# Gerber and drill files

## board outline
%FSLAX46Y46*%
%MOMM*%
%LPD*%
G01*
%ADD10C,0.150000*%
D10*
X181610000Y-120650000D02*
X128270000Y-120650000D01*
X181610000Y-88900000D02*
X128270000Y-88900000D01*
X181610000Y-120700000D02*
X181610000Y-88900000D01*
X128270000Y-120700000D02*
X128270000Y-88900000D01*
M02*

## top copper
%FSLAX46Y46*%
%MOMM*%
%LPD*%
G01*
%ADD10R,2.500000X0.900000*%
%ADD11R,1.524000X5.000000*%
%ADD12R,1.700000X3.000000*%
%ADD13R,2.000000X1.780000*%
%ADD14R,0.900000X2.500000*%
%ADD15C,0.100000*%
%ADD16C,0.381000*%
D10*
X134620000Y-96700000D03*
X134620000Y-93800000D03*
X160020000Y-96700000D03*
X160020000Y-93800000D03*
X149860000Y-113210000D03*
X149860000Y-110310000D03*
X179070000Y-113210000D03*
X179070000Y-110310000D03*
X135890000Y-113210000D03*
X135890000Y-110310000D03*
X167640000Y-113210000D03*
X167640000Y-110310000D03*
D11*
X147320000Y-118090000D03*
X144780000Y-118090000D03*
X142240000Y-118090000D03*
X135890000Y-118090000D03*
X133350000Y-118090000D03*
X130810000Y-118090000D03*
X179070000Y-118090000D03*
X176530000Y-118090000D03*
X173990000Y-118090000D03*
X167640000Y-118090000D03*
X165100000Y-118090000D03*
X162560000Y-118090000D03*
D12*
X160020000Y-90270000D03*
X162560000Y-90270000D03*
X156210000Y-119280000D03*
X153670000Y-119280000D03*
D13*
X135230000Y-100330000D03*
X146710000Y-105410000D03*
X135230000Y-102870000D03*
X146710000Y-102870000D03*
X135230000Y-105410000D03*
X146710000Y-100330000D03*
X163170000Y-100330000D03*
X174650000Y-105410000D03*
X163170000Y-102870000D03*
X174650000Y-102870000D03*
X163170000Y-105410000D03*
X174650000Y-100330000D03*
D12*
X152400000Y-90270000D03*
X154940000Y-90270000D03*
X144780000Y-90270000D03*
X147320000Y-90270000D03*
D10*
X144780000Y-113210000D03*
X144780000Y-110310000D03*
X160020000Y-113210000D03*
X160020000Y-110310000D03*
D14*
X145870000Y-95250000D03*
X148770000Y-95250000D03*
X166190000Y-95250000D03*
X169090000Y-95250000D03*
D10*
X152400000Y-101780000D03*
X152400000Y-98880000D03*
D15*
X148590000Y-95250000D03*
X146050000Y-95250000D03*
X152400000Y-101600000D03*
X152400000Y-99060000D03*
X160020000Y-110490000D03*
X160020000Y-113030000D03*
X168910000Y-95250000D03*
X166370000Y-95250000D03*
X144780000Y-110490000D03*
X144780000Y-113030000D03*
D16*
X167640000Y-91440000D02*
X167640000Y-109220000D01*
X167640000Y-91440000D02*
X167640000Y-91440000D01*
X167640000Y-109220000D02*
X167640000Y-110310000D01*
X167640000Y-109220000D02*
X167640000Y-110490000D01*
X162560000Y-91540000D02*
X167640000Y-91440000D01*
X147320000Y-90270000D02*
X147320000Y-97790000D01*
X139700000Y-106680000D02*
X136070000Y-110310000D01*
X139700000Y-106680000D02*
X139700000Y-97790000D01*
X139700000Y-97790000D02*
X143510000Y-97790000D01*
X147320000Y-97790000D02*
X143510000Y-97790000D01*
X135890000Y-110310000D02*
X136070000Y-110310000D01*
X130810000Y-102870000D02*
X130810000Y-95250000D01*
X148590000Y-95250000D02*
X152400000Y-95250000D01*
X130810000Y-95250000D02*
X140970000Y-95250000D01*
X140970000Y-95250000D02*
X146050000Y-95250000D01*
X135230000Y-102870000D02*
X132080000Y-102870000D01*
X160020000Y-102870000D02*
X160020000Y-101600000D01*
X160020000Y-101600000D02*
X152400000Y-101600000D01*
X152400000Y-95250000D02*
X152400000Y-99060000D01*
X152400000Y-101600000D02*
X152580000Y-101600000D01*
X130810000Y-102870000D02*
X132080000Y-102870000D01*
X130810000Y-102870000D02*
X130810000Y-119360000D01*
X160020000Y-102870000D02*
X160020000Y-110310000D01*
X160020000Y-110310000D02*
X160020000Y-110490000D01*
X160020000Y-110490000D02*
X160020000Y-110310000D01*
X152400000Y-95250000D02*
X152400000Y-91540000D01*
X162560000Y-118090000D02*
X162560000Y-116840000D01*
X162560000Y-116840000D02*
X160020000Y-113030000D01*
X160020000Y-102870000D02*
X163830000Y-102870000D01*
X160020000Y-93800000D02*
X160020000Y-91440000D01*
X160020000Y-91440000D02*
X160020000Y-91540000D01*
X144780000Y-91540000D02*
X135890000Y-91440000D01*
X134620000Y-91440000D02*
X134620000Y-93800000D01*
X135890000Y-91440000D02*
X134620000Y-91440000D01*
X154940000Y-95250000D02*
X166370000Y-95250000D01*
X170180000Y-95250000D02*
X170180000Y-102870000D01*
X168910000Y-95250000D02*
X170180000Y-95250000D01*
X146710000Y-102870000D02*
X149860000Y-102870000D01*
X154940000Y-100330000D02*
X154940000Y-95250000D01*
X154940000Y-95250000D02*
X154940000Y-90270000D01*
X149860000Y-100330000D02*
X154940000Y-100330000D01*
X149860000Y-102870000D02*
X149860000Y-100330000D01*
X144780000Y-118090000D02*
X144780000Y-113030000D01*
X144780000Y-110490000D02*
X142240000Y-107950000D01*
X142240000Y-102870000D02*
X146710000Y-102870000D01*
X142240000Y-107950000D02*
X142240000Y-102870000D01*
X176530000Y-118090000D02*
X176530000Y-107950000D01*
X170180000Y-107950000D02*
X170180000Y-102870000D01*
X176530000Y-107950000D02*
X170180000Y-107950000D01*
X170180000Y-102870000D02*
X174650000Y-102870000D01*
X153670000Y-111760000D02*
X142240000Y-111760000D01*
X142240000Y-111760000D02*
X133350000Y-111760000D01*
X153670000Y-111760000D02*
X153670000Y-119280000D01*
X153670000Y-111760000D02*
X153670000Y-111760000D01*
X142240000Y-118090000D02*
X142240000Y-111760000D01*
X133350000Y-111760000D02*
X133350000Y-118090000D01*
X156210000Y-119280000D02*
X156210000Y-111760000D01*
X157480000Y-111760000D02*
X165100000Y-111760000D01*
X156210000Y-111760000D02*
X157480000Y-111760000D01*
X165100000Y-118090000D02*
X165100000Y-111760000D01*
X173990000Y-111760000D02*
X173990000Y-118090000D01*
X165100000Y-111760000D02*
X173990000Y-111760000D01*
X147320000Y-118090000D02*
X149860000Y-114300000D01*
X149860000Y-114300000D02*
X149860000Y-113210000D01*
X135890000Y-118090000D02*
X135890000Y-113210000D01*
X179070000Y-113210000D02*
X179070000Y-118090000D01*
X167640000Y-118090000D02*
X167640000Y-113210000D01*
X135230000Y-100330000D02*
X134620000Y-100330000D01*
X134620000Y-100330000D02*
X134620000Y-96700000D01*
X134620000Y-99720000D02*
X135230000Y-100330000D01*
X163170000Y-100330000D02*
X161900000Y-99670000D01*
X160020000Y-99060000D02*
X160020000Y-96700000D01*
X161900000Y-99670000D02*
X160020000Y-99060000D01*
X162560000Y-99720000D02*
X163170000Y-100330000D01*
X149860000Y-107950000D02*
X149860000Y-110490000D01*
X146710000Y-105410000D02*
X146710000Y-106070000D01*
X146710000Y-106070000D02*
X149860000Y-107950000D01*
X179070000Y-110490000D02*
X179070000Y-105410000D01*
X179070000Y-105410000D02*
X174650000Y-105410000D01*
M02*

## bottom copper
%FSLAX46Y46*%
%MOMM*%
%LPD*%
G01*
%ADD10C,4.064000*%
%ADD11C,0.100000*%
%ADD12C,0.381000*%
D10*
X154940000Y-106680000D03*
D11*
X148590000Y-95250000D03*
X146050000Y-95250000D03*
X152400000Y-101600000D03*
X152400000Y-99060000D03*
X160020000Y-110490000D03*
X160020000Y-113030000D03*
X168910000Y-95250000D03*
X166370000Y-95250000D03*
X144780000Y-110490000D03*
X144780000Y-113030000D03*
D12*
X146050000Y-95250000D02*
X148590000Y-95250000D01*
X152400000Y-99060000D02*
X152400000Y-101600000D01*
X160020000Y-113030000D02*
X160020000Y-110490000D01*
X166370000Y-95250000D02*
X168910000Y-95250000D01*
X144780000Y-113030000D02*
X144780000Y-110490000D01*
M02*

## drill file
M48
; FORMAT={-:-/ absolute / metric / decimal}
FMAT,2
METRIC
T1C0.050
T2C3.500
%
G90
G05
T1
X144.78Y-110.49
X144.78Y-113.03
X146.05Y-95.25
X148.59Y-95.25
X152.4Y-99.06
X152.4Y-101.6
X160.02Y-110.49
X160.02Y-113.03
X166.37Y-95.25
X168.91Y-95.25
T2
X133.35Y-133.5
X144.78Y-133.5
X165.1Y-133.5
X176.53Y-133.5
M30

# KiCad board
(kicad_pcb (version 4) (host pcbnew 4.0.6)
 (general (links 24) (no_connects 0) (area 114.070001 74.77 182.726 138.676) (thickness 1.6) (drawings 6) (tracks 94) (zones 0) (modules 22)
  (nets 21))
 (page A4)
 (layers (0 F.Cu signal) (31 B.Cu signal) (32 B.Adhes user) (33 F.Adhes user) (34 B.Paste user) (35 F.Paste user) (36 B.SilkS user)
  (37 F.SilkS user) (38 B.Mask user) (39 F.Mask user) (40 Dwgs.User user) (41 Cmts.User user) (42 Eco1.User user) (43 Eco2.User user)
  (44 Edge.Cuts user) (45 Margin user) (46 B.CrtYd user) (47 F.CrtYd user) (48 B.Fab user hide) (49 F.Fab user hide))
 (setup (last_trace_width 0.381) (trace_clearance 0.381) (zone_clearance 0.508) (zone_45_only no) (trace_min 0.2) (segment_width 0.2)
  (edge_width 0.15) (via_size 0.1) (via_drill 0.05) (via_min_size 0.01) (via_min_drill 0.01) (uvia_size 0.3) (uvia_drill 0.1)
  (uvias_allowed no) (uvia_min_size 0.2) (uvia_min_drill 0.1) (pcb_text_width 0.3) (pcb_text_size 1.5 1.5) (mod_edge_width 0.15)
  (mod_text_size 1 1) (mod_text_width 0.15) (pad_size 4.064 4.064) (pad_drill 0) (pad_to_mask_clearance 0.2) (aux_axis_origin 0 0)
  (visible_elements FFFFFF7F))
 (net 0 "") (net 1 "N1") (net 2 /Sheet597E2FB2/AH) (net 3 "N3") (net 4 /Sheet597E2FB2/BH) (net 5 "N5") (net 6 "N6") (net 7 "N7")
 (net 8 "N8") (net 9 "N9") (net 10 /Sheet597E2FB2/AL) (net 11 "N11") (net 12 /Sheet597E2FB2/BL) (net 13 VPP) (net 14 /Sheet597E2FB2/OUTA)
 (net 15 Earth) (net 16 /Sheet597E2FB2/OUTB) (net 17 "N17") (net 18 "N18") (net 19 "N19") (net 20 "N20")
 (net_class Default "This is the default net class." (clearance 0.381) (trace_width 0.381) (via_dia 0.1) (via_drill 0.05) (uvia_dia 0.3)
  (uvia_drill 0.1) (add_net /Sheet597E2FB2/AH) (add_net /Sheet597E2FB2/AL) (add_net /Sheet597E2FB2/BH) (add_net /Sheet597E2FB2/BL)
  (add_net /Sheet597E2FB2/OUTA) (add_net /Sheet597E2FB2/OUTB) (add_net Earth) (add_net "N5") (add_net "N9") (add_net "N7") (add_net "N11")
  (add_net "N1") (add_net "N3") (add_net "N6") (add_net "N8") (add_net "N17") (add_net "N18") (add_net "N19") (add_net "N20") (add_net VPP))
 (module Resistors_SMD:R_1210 (layer F.Cu) (at 134.62 95.25 90)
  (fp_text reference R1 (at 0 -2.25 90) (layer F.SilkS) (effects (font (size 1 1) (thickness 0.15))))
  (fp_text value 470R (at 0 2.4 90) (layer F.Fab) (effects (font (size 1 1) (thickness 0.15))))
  (pad 1 smd rect (at -1.45 0 90) (size 0.9 2.5) (layers F.Cu F.Paste F.Mask) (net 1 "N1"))
  (pad 2 smd rect (at 1.45 0 90) (size 0.9 2.5) (layers F.Cu F.Paste F.Mask) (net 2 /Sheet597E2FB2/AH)))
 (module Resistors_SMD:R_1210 (layer F.Cu) (at 160.02 95.25 90)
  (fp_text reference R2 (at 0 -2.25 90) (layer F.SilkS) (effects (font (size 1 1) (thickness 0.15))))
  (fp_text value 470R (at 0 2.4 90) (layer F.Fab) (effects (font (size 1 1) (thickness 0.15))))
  (pad 1 smd rect (at -1.45 0 90) (size 0.9 2.5) (layers F.Cu F.Paste F.Mask) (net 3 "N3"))
  (pad 2 smd rect (at 1.45 0 90) (size 0.9 2.5) (layers F.Cu F.Paste F.Mask) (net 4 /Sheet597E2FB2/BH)))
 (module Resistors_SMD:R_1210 (layer F.Cu) (at 149.86 111.76 90)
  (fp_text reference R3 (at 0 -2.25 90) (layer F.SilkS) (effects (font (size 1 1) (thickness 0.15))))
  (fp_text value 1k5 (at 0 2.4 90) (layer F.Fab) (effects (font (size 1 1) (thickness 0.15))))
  (pad 1 smd rect (at -1.45 0 90) (size 0.9 2.5) (layers F.Cu F.Paste F.Mask) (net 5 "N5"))
  (pad 2 smd rect (at 1.45 0 90) (size 0.9 2.5) (layers F.Cu F.Paste F.Mask) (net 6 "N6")))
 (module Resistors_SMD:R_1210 (layer F.Cu) (at 179.07 111.76 90)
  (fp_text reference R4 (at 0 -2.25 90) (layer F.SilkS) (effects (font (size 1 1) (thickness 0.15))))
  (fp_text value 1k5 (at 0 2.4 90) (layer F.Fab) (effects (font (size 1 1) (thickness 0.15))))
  (pad 1 smd rect (at -1.45 0 90) (size 0.9 2.5) (layers F.Cu F.Paste F.Mask) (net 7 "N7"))
  (pad 2 smd rect (at 1.45 0 90) (size 0.9 2.5) (layers F.Cu F.Paste F.Mask) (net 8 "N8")))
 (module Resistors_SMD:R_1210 (layer F.Cu) (at 135.89 111.76 90)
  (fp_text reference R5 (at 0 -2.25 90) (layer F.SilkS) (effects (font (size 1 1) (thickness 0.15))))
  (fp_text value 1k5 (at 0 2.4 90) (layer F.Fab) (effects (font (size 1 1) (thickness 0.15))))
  (pad 1 smd rect (at -1.45 0 90) (size 0.9 2.5) (layers F.Cu F.Paste F.Mask) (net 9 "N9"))
  (pad 2 smd rect (at 1.45 0 90) (size 0.9 2.5) (layers F.Cu F.Paste F.Mask) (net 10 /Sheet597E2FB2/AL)))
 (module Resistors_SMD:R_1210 (layer F.Cu) (at 167.64 111.76 90)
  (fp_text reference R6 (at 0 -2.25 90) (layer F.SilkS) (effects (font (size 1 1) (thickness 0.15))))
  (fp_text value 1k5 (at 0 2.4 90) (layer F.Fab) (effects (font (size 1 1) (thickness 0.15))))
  (pad 1 smd rect (at -1.45 0 90) (size 0.9 2.5) (layers F.Cu F.Paste F.Mask) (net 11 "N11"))
  (pad 2 smd rect (at 1.45 0 90) (size 0.9 2.5) (layers F.Cu F.Paste F.Mask) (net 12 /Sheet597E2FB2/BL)))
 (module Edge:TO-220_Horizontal (layer F.Cu) (at 147.32 116.84 180)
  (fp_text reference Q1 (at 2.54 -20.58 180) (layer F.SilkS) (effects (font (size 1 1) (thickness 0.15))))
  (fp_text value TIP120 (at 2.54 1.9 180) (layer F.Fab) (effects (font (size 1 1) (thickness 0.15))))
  (pad 1 smd rect (at 0 -1.25 180) (size 1.524 5) (layers F.Cu F.Paste F.Mask) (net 5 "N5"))
  (pad 2 smd rect (at 2.54 -1.25 180) (size 1.524 5) (layers F.Cu F.Paste F.Mask) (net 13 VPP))
  (pad None np_thru_hole oval (at 2.54 -16.66 180) (size 3.5 3.5) (drill 3.5) (layers *.Cu *.Mask))
  (pad 3 smd rect (at 5.08 -1.25 180) (size 1.524 5) (layers F.Cu F.Paste F.Mask) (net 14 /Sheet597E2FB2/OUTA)))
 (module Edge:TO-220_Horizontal (layer F.Cu) (at 135.89 116.84 180)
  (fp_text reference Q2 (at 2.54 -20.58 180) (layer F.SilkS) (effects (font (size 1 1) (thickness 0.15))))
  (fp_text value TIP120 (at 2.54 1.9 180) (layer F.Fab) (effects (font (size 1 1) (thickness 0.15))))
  (pad 1 smd rect (at 0 -1.25 180) (size 1.524 5) (layers F.Cu F.Paste F.Mask) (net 9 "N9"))
  (pad 2 smd rect (at 2.54 -1.25 180) (size 1.524 5) (layers F.Cu F.Paste F.Mask) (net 14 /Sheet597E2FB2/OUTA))
  (pad None np_thru_hole oval (at 2.54 -16.66 180) (size 3.5 3.5) (drill 3.5) (layers *.Cu *.Mask))
  (pad 3 smd rect (at 5.08 -1.25 180) (size 1.524 5) (layers F.Cu F.Paste F.Mask) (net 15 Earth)))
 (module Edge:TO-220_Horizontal (layer F.Cu) (at 179.07 116.84 180)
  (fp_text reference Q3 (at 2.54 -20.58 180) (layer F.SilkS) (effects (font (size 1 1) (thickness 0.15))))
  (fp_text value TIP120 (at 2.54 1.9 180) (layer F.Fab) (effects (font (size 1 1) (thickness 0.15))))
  (pad 1 smd rect (at 0 -1.25 180) (size 1.524 5) (layers F.Cu F.Paste F.Mask) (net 7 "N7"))
  (pad 2 smd rect (at 2.54 -1.25 180) (size 1.524 5) (layers F.Cu F.Paste F.Mask) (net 13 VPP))
  (pad None np_thru_hole oval (at 2.54 -16.66 180) (size 3.5 3.5) (drill 3.5) (layers *.Cu *.Mask))
  (pad 3 smd rect (at 5.08 -1.25 180) (size 1.524 5) (layers F.Cu F.Paste F.Mask) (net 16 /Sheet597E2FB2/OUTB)))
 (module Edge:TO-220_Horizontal (layer F.Cu) (at 167.64 116.84 180)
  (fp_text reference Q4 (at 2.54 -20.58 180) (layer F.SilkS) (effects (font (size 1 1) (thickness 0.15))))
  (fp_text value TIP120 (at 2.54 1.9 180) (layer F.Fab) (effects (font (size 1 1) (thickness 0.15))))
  (pad 1 smd rect (at 0 -1.25 180) (size 1.524 5) (layers F.Cu F.Paste F.Mask) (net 11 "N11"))
  (pad 2 smd rect (at 2.54 -1.25 180) (size 1.524 5) (layers F.Cu F.Paste F.Mask) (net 16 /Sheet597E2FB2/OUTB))
  (pad None np_thru_hole oval (at 2.54 -16.66 180) (size 3.5 3.5) (drill 3.5) (layers *.Cu *.Mask))
  (pad 3 smd rect (at 5.08 -1.25 180) (size 1.524 5) (layers F.Cu F.Paste F.Mask) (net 15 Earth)))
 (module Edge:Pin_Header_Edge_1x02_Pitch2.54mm (layer F.Cu) (at 160.02 90.17 90)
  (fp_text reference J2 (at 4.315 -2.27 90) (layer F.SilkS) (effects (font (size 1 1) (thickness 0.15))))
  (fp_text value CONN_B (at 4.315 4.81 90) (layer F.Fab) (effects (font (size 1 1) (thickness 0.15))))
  (pad 1 smd rect (at -0.1 0 90) (size 3 1.7) (layers F.Cu F.Paste F.Mask) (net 4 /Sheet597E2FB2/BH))
  (pad 2 smd rect (at -0.1 2.54 90) (size 3 1.7) (layers F.Cu F.Paste F.Mask) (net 12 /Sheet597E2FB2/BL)))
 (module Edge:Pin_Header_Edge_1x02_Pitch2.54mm (layer F.Cu) (at 156.21 119.38 270)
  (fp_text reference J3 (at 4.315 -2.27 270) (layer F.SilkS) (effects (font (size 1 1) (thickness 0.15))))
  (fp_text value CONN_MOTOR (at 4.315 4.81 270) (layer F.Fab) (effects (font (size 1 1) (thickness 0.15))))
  (pad 1 smd rect (at -0.1 0 270) (size 3 1.7) (layers F.Cu F.Paste F.Mask) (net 16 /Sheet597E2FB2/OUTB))
  (pad 2 smd rect (at -0.1 2.54 270) (size 3 1.7) (layers F.Cu F.Paste F.Mask) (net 14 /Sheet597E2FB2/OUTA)))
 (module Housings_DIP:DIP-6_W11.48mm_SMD (layer F.Cu) (at 140.97 102.87)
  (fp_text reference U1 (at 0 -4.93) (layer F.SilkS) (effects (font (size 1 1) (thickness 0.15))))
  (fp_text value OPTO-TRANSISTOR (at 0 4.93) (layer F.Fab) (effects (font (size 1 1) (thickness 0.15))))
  (pad 1 smd rect (at -5.74 -2.54) (size 2 1.78) (layers F.Cu F.Mask) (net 1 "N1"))
  (pad 4 smd rect (at 5.74 2.54) (size 2 1.78) (layers F.Cu F.Mask) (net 6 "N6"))
  (pad 2 smd rect (at -5.74 0) (size 2 1.78) (layers F.Cu F.Mask) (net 15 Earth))
  (pad 5 smd rect (at 5.74 0) (size 2 1.78) (layers F.Cu F.Mask) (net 13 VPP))
  (pad 3 smd rect (at -5.74 2.54) (size 2 1.78) (layers F.Cu F.Mask) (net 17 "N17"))
  (pad 6 smd rect (at 5.74 -2.54) (size 2 1.78) (layers F.Cu F.Mask) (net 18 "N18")))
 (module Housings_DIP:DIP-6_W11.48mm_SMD (layer F.Cu) (at 168.91 102.87)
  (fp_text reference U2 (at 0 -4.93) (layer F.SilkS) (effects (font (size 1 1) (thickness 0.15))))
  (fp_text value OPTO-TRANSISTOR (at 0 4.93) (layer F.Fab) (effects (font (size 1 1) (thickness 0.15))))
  (pad 1 smd rect (at -5.74 -2.54) (size 2 1.78) (layers F.Cu F.Mask) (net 3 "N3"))
  (pad 4 smd rect (at 5.74 2.54) (size 2 1.78) (layers F.Cu F.Mask) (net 8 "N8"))
  (pad 2 smd rect (at -5.74 0) (size 2 1.78) (layers F.Cu F.Mask) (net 15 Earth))
  (pad 5 smd rect (at 5.74 0) (size 2 1.78) (layers F.Cu F.Mask) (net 13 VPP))
  (pad 3 smd rect (at -5.74 2.54) (size 2 1.78) (layers F.Cu F.Mask) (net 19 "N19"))
  (pad 6 smd rect (at 5.74 -2.54) (size 2 1.78) (layers F.Cu F.Mask) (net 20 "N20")))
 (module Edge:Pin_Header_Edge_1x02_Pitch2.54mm (layer F.Cu) (at 152.4 90.17 90)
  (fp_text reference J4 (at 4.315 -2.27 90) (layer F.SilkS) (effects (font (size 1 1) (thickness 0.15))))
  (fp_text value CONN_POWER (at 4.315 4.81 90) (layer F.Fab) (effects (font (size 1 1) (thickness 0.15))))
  (pad 1 smd rect (at -0.1 0 90) (size 3 1.7) (layers F.Cu F.Paste F.Mask) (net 15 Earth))
  (pad 2 smd rect (at -0.1 2.54 90) (size 3 1.7) (layers F.Cu F.Paste F.Mask) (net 13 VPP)))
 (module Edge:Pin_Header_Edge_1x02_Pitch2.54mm (layer F.Cu) (at 144.78 90.17 90)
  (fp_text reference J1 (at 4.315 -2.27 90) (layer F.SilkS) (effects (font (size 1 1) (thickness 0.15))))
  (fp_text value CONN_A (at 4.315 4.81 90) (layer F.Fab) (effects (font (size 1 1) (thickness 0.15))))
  (pad 1 smd rect (at -0.1 0 90) (size 3 1.7) (layers F.Cu F.Paste F.Mask) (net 2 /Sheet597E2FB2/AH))
  (pad 2 smd rect (at -0.1 2.54 90) (size 3 1.7) (layers F.Cu F.Paste F.Mask) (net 10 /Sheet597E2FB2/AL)))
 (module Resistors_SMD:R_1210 (layer F.Cu) (at 144.78 111.76 90)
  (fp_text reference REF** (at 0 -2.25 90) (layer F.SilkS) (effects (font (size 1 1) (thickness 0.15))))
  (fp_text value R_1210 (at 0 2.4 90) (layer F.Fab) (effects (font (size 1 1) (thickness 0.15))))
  (pad 1 smd rect (at -1.45 0 90) (size 0.9 2.5) (layers F.Cu F.Paste F.Mask))
  (pad 2 smd rect (at 1.45 0 90) (size 0.9 2.5) (layers F.Cu F.Paste F.Mask)))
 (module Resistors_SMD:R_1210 (layer F.Cu) (at 160.02 111.76 90)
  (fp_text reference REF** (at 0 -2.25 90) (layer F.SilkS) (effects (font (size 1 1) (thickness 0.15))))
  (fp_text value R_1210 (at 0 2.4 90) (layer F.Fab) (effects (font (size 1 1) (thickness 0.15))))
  (pad 1 smd rect (at -1.45 0 90) (size 0.9 2.5) (layers F.Cu F.Paste F.Mask))
  (pad 2 smd rect (at 1.45 0 90) (size 0.9 2.5) (layers F.Cu F.Paste F.Mask)))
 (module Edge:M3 (layer F.Cu) (at 154.94 106.68)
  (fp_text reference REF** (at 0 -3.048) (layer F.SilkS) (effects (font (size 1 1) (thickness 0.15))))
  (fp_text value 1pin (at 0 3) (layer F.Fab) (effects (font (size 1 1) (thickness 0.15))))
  (pad 1 smd circle (at 0 0) (size 4.064 4.064) (layers B.Cu F.Paste F.Mask)))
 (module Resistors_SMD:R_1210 (layer F.Cu) (at 147.32 95.25)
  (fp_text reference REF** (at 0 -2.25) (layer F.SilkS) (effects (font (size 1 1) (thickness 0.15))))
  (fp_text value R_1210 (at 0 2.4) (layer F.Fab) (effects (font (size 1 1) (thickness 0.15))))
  (pad 1 smd rect (at -1.45 0) (size 0.9 2.5) (layers F.Cu F.Paste F.Mask))
  (pad 2 smd rect (at 1.45 0) (size 0.9 2.5) (layers F.Cu F.Paste F.Mask)))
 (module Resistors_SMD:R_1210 (layer F.Cu) (at 167.64 95.25)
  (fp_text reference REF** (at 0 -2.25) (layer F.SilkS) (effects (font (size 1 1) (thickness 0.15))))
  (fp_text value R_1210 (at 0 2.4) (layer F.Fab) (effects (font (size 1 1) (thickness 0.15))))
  (pad 1 smd rect (at -1.45 0) (size 0.9 2.5) (layers F.Cu F.Paste F.Mask))
  (pad 2 smd rect (at 1.45 0) (size 0.9 2.5) (layers F.Cu F.Paste F.Mask)))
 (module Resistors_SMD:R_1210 (layer F.Cu) (at 152.4 100.33 90)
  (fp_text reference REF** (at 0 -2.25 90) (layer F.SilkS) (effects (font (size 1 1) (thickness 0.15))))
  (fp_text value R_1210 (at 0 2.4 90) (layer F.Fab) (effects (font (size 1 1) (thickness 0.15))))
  (pad 1 smd rect (at -1.45 0 90) (size 0.9 2.5) (layers F.Cu F.Paste F.Mask))
  (pad 2 smd rect (at 1.45 0 90) (size 0.9 2.5) (layers F.Cu F.Paste F.Mask)))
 (gr_line (start 181.61 120.65) (end 128.27 120.65) (angle 90) (layer Edge.Cuts) (width 0.15))
 (gr_line (start 181.61 88.9) (end 128.27 88.9) (angle 90) (layer Edge.Cuts) (width 0.15))
 (gr_line (start 181.61 120.7) (end 181.61 88.9) (angle 90) (layer Edge.Cuts) (width 0.15))
 (gr_line (start 128.27 120.7) (end 128.27 88.9) (angle 90) (layer Edge.Cuts) (width 0.15))
 (segment (start 167.64 91.44) (end 167.64 109.22) (width 0.381) (layer F.Cu) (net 12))
 (segment (start 167.64 91.44) (end 167.64 91.44) (width 0.381) (layer F.Cu) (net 12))
 (segment (start 167.64 109.22) (end 167.64 110.31) (width 0.381) (layer F.Cu) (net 12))
 (segment (start 167.64 109.22) (end 167.64 110.49) (width 0.381) (layer F.Cu) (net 12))
 (segment (start 162.56 91.54) (end 167.64 91.44) (width 0.381) (layer F.Cu) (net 12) (status 10))
 (segment (start 147.32 90.27) (end 147.32 97.79) (width 0.381) (layer F.Cu) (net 10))
 (segment (start 139.7 106.68) (end 136.07 110.31) (width 0.381) (layer F.Cu) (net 10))
 (segment (start 139.7 106.68) (end 139.7 97.79) (width 0.381) (layer F.Cu) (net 10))
 (segment (start 139.7 97.79) (end 143.51 97.79) (width 0.381) (layer F.Cu) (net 10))
 (segment (start 147.32 97.79) (end 143.51 97.79) (width 0.381) (layer F.Cu) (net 10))
 (segment (start 135.89 110.31) (end 136.07 110.31) (width 0.381) (layer F.Cu) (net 10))
 (segment (start 130.81 102.87) (end 130.81 95.25) (width 0.381) (layer F.Cu) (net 15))
 (via (at 148.59 95.25) (size 0.1) (drill 0.05) (layers F.Cu B.Cu) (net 15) (status 30))
 (segment (start 148.59 95.25) (end 152.4 95.25) (width 0.381) (layer F.Cu) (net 15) (status 10))
 (segment (start 130.81 95.25) (end 140.97 95.25) (width 0.381) (layer F.Cu) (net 15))
 (segment (start 140.97 95.25) (end 146.05 95.25) (width 0.381) (layer F.Cu) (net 15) (status 20))
 (via (at 146.05 95.25) (size 0.1) (drill 0.05) (layers F.Cu B.Cu) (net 15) (status 30))
 (segment (start 146.05 95.25) (end 148.59 95.25) (width 0.381) (layer B.Cu) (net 15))
 (segment (start 135.23 102.87) (end 132.08 102.87) (width 0.381) (layer F.Cu) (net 15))
 (segment (start 160.02 102.87) (end 160.02 101.6) (width 0.381) (layer F.Cu) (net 15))
 (segment (start 160.02 101.6) (end 152.4 101.6) (width 0.381) (layer F.Cu) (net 15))
 (segment (start 152.4 95.25) (end 152.4 99.06) (width 0.381) (layer F.Cu) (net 15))
 (via (at 152.4 101.6) (size 0.1) (drill 0.05) (layers F.Cu B.Cu) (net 15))
 (segment (start 152.4 99.06) (end 152.4 101.6) (width 0.381) (layer B.Cu) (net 15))
 (via (at 152.4 99.06) (size 0.1) (drill 0.05) (layers F.Cu B.Cu) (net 15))
 (segment (start 152.4 101.6) (end 152.58 101.6) (width 0.381) (layer F.Cu) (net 15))
 (segment (start 130.81 102.87) (end 132.08 102.87) (width 0.381) (layer F.Cu) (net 15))
 (segment (start 130.81 102.87) (end 130.81 119.36) (width 0.381) (layer F.Cu) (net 15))
 (segment (start 160.02 102.87) (end 160.02 110.31) (width 0.381) (layer F.Cu) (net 15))
 (segment (start 160.02 110.31) (end 160.02 110.49) (width 0.381) (layer F.Cu) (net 15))
 (segment (start 160.02 110.49) (end 160.02 110.31) (width 0.381) (layer F.Cu) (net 15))
 (segment (start 152.4 95.25) (end 152.4 91.54) (width 0.381) (layer F.Cu) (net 15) (status 20))
 (segment (start 162.56 118.09) (end 162.56 116.84) (width 0.381) (layer F.Cu) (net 15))
 (segment (start 162.56 116.84) (end 160.02 113.03) (width 0.381) (layer F.Cu) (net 15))
 (via (at 160.02 110.49) (size 0.1) (drill 0.05) (layers F.Cu B.Cu) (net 15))
 (segment (start 160.02 113.03) (end 160.02 110.49) (width 0.381) (layer B.Cu) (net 15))
 (via (at 160.02 113.03) (size 0.1) (drill 0.05) (layers F.Cu B.Cu) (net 15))
 (segment (start 160.02 102.87) (end 163.83 102.87) (width 0.381) (layer F.Cu) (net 15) (status 20))
 (segment (start 160.02 93.8) (end 160.02 91.44) (width 0.381) (layer F.Cu) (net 4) (status 10))
 (segment (start 160.02 91.44) (end 160.02 91.54) (width 0.381) (layer F.Cu) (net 4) (status 30))
 (segment (start 144.78 91.54) (end 135.89 91.44) (width 0.381) (layer F.Cu) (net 2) (status 10))
 (segment (start 134.62 91.44) (end 134.62 93.8) (width 0.381) (layer F.Cu) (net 2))
 (segment (start 135.89 91.44) (end 134.62 91.44) (width 0.381) (layer F.Cu) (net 2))
 (segment (start 154.94 95.25) (end 166.37 95.25) (width 0.381) (layer F.Cu) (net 13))
 (segment (start 170.18 95.25) (end 170.18 102.87) (width 0.381) (layer F.Cu) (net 13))
 (segment (start 168.91 95.25) (end 170.18 95.25) (width 0.381) (layer F.Cu) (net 13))
 (via (at 168.91 95.25) (size 0.1) (drill 0.05) (layers F.Cu B.Cu) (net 13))
 (segment (start 166.37 95.25) (end 168.91 95.25) (width 0.381) (layer B.Cu) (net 13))
 (via (at 166.37 95.25) (size 0.1) (drill 0.05) (layers F.Cu B.Cu) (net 13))
 (segment (start 146.71 102.87) (end 149.86 102.87) (width 0.381) (layer F.Cu) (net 13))
 (segment (start 154.94 100.33) (end 154.94 95.25) (width 0.381) (layer F.Cu) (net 13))
 (segment (start 154.94 95.25) (end 154.94 90.27) (width 0.381) (layer F.Cu) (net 13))
 (segment (start 149.86 100.33) (end 154.94 100.33) (width 0.381) (layer F.Cu) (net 13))
 (segment (start 149.86 102.87) (end 149.86 100.33) (width 0.381) (layer F.Cu) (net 13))
 (segment (start 144.78 118.09) (end 144.78 113.03) (width 0.381) (layer F.Cu) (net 13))
 (via (at 144.78 110.49) (size 0.1) (drill 0.05) (layers F.Cu B.Cu) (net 13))
 (segment (start 144.78 113.03) (end 144.78 110.49) (width 0.381) (layer B.Cu) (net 13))
 (via (at 144.78 113.03) (size 0.1) (drill 0.05) (layers F.Cu B.Cu) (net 13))
 (segment (start 144.78 110.49) (end 142.24 107.95) (width 0.381) (layer F.Cu) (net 13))
 (segment (start 142.24 102.87) (end 146.71 102.87) (width 0.381) (layer F.Cu) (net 13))
 (segment (start 142.24 107.95) (end 142.24 102.87) (width 0.381) (layer F.Cu) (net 13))
 (segment (start 176.53 118.09) (end 176.53 107.95) (width 0.381) (layer F.Cu) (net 13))
 (segment (start 170.18 107.95) (end 170.18 102.87) (width 0.381) (layer F.Cu) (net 13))
 (segment (start 176.53 107.95) (end 170.18 107.95) (width 0.381) (layer F.Cu) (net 13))
 (segment (start 170.18 102.87) (end 174.65 102.87) (width 0.381) (layer F.Cu) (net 13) (status 20))
 (segment (start 153.67 111.76) (end 142.24 111.76) (width 0.381) (layer F.Cu) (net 14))
 (segment (start 142.24 111.76) (end 133.35 111.76) (width 0.381) (layer F.Cu) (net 14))
 (segment (start 153.67 111.76) (end 153.67 119.28) (width 0.381) (layer F.Cu) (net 14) (status 20))
 (segment (start 153.67 111.76) (end 153.67 111.76) (width 0.381) (layer F.Cu) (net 14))
 (segment (start 142.24 118.09) (end 142.24 111.76) (width 0.381) (layer F.Cu) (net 14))
 (segment (start 133.35 111.76) (end 133.35 118.09) (width 0.381) (layer F.Cu) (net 14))
 (segment (start 156.21 119.28) (end 156.21 111.76) (width 0.381) (layer F.Cu) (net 16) (status 10))
 (segment (start 157.48 111.76) (end 165.1 111.76) (width 0.381) (layer F.Cu) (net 16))
 (segment (start 156.21 111.76) (end 157.48 111.76) (width 0.381) (layer F.Cu) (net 16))
 (segment (start 165.1 118.09) (end 165.1 111.76) (width 0.381) (layer F.Cu) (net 16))
 (segment (start 173.99 111.76) (end 173.99 118.09) (width 0.381) (layer F.Cu) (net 16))
 (segment (start 165.1 111.76) (end 173.99 111.76) (width 0.381) (layer F.Cu) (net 16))
 (segment (start 147.32 118.09) (end 149.86 114.3) (width 0.381) (layer F.Cu) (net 5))
 (segment (start 149.86 114.3) (end 149.86 113.21) (width 0.381) (layer F.Cu) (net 5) (status 20))
 (segment (start 135.89 118.09) (end 135.89 113.21) (width 0.381) (layer F.Cu) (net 9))
 (segment (start 179.07 113.21) (end 179.07 118.09) (width 0.381) (layer F.Cu) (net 7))
 (segment (start 167.64 118.09) (end 167.64 113.21) (width 0.381) (layer F.Cu) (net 11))
 (segment (start 135.23 100.33) (end 134.62 100.33) (width 0.381) (layer F.Cu) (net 1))
 (segment (start 134.62 100.33) (end 134.62 96.7) (width 0.381) (layer F.Cu) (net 1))
 (segment (start 134.62 99.72) (end 135.23 100.33) (width 0.381) (layer F.Cu) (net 1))
 (segment (start 163.17 100.33) (end 161.9 99.67) (width 0.381) (layer F.Cu) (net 3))
 (segment (start 160.02 99.06) (end 160.02 96.7) (width 0.381) (layer F.Cu) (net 3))
 (segment (start 161.9 99.67) (end 160.02 99.06) (width 0.381) (layer F.Cu) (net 3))
 (segment (start 162.56 99.72) (end 163.17 100.33) (width 0.381) (layer F.Cu) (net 3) (status 30))
 (segment (start 149.86 107.95) (end 149.86 110.49) (width 0.381) (layer F.Cu) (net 6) (status 20))
 (segment (start 146.71 105.41) (end 146.71 106.07) (width 0.381) (layer F.Cu) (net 6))
 (segment (start 146.71 106.07) (end 149.86 107.95) (width 0.381) (layer F.Cu) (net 6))
 (segment (start 179.07 110.49) (end 179.07 105.41) (width 0.381) (layer F.Cu) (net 8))
 (segment (start 179.07 105.41) (end 174.65 105.41) (width 0.381) (layer F.Cu) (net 8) (status 20)))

